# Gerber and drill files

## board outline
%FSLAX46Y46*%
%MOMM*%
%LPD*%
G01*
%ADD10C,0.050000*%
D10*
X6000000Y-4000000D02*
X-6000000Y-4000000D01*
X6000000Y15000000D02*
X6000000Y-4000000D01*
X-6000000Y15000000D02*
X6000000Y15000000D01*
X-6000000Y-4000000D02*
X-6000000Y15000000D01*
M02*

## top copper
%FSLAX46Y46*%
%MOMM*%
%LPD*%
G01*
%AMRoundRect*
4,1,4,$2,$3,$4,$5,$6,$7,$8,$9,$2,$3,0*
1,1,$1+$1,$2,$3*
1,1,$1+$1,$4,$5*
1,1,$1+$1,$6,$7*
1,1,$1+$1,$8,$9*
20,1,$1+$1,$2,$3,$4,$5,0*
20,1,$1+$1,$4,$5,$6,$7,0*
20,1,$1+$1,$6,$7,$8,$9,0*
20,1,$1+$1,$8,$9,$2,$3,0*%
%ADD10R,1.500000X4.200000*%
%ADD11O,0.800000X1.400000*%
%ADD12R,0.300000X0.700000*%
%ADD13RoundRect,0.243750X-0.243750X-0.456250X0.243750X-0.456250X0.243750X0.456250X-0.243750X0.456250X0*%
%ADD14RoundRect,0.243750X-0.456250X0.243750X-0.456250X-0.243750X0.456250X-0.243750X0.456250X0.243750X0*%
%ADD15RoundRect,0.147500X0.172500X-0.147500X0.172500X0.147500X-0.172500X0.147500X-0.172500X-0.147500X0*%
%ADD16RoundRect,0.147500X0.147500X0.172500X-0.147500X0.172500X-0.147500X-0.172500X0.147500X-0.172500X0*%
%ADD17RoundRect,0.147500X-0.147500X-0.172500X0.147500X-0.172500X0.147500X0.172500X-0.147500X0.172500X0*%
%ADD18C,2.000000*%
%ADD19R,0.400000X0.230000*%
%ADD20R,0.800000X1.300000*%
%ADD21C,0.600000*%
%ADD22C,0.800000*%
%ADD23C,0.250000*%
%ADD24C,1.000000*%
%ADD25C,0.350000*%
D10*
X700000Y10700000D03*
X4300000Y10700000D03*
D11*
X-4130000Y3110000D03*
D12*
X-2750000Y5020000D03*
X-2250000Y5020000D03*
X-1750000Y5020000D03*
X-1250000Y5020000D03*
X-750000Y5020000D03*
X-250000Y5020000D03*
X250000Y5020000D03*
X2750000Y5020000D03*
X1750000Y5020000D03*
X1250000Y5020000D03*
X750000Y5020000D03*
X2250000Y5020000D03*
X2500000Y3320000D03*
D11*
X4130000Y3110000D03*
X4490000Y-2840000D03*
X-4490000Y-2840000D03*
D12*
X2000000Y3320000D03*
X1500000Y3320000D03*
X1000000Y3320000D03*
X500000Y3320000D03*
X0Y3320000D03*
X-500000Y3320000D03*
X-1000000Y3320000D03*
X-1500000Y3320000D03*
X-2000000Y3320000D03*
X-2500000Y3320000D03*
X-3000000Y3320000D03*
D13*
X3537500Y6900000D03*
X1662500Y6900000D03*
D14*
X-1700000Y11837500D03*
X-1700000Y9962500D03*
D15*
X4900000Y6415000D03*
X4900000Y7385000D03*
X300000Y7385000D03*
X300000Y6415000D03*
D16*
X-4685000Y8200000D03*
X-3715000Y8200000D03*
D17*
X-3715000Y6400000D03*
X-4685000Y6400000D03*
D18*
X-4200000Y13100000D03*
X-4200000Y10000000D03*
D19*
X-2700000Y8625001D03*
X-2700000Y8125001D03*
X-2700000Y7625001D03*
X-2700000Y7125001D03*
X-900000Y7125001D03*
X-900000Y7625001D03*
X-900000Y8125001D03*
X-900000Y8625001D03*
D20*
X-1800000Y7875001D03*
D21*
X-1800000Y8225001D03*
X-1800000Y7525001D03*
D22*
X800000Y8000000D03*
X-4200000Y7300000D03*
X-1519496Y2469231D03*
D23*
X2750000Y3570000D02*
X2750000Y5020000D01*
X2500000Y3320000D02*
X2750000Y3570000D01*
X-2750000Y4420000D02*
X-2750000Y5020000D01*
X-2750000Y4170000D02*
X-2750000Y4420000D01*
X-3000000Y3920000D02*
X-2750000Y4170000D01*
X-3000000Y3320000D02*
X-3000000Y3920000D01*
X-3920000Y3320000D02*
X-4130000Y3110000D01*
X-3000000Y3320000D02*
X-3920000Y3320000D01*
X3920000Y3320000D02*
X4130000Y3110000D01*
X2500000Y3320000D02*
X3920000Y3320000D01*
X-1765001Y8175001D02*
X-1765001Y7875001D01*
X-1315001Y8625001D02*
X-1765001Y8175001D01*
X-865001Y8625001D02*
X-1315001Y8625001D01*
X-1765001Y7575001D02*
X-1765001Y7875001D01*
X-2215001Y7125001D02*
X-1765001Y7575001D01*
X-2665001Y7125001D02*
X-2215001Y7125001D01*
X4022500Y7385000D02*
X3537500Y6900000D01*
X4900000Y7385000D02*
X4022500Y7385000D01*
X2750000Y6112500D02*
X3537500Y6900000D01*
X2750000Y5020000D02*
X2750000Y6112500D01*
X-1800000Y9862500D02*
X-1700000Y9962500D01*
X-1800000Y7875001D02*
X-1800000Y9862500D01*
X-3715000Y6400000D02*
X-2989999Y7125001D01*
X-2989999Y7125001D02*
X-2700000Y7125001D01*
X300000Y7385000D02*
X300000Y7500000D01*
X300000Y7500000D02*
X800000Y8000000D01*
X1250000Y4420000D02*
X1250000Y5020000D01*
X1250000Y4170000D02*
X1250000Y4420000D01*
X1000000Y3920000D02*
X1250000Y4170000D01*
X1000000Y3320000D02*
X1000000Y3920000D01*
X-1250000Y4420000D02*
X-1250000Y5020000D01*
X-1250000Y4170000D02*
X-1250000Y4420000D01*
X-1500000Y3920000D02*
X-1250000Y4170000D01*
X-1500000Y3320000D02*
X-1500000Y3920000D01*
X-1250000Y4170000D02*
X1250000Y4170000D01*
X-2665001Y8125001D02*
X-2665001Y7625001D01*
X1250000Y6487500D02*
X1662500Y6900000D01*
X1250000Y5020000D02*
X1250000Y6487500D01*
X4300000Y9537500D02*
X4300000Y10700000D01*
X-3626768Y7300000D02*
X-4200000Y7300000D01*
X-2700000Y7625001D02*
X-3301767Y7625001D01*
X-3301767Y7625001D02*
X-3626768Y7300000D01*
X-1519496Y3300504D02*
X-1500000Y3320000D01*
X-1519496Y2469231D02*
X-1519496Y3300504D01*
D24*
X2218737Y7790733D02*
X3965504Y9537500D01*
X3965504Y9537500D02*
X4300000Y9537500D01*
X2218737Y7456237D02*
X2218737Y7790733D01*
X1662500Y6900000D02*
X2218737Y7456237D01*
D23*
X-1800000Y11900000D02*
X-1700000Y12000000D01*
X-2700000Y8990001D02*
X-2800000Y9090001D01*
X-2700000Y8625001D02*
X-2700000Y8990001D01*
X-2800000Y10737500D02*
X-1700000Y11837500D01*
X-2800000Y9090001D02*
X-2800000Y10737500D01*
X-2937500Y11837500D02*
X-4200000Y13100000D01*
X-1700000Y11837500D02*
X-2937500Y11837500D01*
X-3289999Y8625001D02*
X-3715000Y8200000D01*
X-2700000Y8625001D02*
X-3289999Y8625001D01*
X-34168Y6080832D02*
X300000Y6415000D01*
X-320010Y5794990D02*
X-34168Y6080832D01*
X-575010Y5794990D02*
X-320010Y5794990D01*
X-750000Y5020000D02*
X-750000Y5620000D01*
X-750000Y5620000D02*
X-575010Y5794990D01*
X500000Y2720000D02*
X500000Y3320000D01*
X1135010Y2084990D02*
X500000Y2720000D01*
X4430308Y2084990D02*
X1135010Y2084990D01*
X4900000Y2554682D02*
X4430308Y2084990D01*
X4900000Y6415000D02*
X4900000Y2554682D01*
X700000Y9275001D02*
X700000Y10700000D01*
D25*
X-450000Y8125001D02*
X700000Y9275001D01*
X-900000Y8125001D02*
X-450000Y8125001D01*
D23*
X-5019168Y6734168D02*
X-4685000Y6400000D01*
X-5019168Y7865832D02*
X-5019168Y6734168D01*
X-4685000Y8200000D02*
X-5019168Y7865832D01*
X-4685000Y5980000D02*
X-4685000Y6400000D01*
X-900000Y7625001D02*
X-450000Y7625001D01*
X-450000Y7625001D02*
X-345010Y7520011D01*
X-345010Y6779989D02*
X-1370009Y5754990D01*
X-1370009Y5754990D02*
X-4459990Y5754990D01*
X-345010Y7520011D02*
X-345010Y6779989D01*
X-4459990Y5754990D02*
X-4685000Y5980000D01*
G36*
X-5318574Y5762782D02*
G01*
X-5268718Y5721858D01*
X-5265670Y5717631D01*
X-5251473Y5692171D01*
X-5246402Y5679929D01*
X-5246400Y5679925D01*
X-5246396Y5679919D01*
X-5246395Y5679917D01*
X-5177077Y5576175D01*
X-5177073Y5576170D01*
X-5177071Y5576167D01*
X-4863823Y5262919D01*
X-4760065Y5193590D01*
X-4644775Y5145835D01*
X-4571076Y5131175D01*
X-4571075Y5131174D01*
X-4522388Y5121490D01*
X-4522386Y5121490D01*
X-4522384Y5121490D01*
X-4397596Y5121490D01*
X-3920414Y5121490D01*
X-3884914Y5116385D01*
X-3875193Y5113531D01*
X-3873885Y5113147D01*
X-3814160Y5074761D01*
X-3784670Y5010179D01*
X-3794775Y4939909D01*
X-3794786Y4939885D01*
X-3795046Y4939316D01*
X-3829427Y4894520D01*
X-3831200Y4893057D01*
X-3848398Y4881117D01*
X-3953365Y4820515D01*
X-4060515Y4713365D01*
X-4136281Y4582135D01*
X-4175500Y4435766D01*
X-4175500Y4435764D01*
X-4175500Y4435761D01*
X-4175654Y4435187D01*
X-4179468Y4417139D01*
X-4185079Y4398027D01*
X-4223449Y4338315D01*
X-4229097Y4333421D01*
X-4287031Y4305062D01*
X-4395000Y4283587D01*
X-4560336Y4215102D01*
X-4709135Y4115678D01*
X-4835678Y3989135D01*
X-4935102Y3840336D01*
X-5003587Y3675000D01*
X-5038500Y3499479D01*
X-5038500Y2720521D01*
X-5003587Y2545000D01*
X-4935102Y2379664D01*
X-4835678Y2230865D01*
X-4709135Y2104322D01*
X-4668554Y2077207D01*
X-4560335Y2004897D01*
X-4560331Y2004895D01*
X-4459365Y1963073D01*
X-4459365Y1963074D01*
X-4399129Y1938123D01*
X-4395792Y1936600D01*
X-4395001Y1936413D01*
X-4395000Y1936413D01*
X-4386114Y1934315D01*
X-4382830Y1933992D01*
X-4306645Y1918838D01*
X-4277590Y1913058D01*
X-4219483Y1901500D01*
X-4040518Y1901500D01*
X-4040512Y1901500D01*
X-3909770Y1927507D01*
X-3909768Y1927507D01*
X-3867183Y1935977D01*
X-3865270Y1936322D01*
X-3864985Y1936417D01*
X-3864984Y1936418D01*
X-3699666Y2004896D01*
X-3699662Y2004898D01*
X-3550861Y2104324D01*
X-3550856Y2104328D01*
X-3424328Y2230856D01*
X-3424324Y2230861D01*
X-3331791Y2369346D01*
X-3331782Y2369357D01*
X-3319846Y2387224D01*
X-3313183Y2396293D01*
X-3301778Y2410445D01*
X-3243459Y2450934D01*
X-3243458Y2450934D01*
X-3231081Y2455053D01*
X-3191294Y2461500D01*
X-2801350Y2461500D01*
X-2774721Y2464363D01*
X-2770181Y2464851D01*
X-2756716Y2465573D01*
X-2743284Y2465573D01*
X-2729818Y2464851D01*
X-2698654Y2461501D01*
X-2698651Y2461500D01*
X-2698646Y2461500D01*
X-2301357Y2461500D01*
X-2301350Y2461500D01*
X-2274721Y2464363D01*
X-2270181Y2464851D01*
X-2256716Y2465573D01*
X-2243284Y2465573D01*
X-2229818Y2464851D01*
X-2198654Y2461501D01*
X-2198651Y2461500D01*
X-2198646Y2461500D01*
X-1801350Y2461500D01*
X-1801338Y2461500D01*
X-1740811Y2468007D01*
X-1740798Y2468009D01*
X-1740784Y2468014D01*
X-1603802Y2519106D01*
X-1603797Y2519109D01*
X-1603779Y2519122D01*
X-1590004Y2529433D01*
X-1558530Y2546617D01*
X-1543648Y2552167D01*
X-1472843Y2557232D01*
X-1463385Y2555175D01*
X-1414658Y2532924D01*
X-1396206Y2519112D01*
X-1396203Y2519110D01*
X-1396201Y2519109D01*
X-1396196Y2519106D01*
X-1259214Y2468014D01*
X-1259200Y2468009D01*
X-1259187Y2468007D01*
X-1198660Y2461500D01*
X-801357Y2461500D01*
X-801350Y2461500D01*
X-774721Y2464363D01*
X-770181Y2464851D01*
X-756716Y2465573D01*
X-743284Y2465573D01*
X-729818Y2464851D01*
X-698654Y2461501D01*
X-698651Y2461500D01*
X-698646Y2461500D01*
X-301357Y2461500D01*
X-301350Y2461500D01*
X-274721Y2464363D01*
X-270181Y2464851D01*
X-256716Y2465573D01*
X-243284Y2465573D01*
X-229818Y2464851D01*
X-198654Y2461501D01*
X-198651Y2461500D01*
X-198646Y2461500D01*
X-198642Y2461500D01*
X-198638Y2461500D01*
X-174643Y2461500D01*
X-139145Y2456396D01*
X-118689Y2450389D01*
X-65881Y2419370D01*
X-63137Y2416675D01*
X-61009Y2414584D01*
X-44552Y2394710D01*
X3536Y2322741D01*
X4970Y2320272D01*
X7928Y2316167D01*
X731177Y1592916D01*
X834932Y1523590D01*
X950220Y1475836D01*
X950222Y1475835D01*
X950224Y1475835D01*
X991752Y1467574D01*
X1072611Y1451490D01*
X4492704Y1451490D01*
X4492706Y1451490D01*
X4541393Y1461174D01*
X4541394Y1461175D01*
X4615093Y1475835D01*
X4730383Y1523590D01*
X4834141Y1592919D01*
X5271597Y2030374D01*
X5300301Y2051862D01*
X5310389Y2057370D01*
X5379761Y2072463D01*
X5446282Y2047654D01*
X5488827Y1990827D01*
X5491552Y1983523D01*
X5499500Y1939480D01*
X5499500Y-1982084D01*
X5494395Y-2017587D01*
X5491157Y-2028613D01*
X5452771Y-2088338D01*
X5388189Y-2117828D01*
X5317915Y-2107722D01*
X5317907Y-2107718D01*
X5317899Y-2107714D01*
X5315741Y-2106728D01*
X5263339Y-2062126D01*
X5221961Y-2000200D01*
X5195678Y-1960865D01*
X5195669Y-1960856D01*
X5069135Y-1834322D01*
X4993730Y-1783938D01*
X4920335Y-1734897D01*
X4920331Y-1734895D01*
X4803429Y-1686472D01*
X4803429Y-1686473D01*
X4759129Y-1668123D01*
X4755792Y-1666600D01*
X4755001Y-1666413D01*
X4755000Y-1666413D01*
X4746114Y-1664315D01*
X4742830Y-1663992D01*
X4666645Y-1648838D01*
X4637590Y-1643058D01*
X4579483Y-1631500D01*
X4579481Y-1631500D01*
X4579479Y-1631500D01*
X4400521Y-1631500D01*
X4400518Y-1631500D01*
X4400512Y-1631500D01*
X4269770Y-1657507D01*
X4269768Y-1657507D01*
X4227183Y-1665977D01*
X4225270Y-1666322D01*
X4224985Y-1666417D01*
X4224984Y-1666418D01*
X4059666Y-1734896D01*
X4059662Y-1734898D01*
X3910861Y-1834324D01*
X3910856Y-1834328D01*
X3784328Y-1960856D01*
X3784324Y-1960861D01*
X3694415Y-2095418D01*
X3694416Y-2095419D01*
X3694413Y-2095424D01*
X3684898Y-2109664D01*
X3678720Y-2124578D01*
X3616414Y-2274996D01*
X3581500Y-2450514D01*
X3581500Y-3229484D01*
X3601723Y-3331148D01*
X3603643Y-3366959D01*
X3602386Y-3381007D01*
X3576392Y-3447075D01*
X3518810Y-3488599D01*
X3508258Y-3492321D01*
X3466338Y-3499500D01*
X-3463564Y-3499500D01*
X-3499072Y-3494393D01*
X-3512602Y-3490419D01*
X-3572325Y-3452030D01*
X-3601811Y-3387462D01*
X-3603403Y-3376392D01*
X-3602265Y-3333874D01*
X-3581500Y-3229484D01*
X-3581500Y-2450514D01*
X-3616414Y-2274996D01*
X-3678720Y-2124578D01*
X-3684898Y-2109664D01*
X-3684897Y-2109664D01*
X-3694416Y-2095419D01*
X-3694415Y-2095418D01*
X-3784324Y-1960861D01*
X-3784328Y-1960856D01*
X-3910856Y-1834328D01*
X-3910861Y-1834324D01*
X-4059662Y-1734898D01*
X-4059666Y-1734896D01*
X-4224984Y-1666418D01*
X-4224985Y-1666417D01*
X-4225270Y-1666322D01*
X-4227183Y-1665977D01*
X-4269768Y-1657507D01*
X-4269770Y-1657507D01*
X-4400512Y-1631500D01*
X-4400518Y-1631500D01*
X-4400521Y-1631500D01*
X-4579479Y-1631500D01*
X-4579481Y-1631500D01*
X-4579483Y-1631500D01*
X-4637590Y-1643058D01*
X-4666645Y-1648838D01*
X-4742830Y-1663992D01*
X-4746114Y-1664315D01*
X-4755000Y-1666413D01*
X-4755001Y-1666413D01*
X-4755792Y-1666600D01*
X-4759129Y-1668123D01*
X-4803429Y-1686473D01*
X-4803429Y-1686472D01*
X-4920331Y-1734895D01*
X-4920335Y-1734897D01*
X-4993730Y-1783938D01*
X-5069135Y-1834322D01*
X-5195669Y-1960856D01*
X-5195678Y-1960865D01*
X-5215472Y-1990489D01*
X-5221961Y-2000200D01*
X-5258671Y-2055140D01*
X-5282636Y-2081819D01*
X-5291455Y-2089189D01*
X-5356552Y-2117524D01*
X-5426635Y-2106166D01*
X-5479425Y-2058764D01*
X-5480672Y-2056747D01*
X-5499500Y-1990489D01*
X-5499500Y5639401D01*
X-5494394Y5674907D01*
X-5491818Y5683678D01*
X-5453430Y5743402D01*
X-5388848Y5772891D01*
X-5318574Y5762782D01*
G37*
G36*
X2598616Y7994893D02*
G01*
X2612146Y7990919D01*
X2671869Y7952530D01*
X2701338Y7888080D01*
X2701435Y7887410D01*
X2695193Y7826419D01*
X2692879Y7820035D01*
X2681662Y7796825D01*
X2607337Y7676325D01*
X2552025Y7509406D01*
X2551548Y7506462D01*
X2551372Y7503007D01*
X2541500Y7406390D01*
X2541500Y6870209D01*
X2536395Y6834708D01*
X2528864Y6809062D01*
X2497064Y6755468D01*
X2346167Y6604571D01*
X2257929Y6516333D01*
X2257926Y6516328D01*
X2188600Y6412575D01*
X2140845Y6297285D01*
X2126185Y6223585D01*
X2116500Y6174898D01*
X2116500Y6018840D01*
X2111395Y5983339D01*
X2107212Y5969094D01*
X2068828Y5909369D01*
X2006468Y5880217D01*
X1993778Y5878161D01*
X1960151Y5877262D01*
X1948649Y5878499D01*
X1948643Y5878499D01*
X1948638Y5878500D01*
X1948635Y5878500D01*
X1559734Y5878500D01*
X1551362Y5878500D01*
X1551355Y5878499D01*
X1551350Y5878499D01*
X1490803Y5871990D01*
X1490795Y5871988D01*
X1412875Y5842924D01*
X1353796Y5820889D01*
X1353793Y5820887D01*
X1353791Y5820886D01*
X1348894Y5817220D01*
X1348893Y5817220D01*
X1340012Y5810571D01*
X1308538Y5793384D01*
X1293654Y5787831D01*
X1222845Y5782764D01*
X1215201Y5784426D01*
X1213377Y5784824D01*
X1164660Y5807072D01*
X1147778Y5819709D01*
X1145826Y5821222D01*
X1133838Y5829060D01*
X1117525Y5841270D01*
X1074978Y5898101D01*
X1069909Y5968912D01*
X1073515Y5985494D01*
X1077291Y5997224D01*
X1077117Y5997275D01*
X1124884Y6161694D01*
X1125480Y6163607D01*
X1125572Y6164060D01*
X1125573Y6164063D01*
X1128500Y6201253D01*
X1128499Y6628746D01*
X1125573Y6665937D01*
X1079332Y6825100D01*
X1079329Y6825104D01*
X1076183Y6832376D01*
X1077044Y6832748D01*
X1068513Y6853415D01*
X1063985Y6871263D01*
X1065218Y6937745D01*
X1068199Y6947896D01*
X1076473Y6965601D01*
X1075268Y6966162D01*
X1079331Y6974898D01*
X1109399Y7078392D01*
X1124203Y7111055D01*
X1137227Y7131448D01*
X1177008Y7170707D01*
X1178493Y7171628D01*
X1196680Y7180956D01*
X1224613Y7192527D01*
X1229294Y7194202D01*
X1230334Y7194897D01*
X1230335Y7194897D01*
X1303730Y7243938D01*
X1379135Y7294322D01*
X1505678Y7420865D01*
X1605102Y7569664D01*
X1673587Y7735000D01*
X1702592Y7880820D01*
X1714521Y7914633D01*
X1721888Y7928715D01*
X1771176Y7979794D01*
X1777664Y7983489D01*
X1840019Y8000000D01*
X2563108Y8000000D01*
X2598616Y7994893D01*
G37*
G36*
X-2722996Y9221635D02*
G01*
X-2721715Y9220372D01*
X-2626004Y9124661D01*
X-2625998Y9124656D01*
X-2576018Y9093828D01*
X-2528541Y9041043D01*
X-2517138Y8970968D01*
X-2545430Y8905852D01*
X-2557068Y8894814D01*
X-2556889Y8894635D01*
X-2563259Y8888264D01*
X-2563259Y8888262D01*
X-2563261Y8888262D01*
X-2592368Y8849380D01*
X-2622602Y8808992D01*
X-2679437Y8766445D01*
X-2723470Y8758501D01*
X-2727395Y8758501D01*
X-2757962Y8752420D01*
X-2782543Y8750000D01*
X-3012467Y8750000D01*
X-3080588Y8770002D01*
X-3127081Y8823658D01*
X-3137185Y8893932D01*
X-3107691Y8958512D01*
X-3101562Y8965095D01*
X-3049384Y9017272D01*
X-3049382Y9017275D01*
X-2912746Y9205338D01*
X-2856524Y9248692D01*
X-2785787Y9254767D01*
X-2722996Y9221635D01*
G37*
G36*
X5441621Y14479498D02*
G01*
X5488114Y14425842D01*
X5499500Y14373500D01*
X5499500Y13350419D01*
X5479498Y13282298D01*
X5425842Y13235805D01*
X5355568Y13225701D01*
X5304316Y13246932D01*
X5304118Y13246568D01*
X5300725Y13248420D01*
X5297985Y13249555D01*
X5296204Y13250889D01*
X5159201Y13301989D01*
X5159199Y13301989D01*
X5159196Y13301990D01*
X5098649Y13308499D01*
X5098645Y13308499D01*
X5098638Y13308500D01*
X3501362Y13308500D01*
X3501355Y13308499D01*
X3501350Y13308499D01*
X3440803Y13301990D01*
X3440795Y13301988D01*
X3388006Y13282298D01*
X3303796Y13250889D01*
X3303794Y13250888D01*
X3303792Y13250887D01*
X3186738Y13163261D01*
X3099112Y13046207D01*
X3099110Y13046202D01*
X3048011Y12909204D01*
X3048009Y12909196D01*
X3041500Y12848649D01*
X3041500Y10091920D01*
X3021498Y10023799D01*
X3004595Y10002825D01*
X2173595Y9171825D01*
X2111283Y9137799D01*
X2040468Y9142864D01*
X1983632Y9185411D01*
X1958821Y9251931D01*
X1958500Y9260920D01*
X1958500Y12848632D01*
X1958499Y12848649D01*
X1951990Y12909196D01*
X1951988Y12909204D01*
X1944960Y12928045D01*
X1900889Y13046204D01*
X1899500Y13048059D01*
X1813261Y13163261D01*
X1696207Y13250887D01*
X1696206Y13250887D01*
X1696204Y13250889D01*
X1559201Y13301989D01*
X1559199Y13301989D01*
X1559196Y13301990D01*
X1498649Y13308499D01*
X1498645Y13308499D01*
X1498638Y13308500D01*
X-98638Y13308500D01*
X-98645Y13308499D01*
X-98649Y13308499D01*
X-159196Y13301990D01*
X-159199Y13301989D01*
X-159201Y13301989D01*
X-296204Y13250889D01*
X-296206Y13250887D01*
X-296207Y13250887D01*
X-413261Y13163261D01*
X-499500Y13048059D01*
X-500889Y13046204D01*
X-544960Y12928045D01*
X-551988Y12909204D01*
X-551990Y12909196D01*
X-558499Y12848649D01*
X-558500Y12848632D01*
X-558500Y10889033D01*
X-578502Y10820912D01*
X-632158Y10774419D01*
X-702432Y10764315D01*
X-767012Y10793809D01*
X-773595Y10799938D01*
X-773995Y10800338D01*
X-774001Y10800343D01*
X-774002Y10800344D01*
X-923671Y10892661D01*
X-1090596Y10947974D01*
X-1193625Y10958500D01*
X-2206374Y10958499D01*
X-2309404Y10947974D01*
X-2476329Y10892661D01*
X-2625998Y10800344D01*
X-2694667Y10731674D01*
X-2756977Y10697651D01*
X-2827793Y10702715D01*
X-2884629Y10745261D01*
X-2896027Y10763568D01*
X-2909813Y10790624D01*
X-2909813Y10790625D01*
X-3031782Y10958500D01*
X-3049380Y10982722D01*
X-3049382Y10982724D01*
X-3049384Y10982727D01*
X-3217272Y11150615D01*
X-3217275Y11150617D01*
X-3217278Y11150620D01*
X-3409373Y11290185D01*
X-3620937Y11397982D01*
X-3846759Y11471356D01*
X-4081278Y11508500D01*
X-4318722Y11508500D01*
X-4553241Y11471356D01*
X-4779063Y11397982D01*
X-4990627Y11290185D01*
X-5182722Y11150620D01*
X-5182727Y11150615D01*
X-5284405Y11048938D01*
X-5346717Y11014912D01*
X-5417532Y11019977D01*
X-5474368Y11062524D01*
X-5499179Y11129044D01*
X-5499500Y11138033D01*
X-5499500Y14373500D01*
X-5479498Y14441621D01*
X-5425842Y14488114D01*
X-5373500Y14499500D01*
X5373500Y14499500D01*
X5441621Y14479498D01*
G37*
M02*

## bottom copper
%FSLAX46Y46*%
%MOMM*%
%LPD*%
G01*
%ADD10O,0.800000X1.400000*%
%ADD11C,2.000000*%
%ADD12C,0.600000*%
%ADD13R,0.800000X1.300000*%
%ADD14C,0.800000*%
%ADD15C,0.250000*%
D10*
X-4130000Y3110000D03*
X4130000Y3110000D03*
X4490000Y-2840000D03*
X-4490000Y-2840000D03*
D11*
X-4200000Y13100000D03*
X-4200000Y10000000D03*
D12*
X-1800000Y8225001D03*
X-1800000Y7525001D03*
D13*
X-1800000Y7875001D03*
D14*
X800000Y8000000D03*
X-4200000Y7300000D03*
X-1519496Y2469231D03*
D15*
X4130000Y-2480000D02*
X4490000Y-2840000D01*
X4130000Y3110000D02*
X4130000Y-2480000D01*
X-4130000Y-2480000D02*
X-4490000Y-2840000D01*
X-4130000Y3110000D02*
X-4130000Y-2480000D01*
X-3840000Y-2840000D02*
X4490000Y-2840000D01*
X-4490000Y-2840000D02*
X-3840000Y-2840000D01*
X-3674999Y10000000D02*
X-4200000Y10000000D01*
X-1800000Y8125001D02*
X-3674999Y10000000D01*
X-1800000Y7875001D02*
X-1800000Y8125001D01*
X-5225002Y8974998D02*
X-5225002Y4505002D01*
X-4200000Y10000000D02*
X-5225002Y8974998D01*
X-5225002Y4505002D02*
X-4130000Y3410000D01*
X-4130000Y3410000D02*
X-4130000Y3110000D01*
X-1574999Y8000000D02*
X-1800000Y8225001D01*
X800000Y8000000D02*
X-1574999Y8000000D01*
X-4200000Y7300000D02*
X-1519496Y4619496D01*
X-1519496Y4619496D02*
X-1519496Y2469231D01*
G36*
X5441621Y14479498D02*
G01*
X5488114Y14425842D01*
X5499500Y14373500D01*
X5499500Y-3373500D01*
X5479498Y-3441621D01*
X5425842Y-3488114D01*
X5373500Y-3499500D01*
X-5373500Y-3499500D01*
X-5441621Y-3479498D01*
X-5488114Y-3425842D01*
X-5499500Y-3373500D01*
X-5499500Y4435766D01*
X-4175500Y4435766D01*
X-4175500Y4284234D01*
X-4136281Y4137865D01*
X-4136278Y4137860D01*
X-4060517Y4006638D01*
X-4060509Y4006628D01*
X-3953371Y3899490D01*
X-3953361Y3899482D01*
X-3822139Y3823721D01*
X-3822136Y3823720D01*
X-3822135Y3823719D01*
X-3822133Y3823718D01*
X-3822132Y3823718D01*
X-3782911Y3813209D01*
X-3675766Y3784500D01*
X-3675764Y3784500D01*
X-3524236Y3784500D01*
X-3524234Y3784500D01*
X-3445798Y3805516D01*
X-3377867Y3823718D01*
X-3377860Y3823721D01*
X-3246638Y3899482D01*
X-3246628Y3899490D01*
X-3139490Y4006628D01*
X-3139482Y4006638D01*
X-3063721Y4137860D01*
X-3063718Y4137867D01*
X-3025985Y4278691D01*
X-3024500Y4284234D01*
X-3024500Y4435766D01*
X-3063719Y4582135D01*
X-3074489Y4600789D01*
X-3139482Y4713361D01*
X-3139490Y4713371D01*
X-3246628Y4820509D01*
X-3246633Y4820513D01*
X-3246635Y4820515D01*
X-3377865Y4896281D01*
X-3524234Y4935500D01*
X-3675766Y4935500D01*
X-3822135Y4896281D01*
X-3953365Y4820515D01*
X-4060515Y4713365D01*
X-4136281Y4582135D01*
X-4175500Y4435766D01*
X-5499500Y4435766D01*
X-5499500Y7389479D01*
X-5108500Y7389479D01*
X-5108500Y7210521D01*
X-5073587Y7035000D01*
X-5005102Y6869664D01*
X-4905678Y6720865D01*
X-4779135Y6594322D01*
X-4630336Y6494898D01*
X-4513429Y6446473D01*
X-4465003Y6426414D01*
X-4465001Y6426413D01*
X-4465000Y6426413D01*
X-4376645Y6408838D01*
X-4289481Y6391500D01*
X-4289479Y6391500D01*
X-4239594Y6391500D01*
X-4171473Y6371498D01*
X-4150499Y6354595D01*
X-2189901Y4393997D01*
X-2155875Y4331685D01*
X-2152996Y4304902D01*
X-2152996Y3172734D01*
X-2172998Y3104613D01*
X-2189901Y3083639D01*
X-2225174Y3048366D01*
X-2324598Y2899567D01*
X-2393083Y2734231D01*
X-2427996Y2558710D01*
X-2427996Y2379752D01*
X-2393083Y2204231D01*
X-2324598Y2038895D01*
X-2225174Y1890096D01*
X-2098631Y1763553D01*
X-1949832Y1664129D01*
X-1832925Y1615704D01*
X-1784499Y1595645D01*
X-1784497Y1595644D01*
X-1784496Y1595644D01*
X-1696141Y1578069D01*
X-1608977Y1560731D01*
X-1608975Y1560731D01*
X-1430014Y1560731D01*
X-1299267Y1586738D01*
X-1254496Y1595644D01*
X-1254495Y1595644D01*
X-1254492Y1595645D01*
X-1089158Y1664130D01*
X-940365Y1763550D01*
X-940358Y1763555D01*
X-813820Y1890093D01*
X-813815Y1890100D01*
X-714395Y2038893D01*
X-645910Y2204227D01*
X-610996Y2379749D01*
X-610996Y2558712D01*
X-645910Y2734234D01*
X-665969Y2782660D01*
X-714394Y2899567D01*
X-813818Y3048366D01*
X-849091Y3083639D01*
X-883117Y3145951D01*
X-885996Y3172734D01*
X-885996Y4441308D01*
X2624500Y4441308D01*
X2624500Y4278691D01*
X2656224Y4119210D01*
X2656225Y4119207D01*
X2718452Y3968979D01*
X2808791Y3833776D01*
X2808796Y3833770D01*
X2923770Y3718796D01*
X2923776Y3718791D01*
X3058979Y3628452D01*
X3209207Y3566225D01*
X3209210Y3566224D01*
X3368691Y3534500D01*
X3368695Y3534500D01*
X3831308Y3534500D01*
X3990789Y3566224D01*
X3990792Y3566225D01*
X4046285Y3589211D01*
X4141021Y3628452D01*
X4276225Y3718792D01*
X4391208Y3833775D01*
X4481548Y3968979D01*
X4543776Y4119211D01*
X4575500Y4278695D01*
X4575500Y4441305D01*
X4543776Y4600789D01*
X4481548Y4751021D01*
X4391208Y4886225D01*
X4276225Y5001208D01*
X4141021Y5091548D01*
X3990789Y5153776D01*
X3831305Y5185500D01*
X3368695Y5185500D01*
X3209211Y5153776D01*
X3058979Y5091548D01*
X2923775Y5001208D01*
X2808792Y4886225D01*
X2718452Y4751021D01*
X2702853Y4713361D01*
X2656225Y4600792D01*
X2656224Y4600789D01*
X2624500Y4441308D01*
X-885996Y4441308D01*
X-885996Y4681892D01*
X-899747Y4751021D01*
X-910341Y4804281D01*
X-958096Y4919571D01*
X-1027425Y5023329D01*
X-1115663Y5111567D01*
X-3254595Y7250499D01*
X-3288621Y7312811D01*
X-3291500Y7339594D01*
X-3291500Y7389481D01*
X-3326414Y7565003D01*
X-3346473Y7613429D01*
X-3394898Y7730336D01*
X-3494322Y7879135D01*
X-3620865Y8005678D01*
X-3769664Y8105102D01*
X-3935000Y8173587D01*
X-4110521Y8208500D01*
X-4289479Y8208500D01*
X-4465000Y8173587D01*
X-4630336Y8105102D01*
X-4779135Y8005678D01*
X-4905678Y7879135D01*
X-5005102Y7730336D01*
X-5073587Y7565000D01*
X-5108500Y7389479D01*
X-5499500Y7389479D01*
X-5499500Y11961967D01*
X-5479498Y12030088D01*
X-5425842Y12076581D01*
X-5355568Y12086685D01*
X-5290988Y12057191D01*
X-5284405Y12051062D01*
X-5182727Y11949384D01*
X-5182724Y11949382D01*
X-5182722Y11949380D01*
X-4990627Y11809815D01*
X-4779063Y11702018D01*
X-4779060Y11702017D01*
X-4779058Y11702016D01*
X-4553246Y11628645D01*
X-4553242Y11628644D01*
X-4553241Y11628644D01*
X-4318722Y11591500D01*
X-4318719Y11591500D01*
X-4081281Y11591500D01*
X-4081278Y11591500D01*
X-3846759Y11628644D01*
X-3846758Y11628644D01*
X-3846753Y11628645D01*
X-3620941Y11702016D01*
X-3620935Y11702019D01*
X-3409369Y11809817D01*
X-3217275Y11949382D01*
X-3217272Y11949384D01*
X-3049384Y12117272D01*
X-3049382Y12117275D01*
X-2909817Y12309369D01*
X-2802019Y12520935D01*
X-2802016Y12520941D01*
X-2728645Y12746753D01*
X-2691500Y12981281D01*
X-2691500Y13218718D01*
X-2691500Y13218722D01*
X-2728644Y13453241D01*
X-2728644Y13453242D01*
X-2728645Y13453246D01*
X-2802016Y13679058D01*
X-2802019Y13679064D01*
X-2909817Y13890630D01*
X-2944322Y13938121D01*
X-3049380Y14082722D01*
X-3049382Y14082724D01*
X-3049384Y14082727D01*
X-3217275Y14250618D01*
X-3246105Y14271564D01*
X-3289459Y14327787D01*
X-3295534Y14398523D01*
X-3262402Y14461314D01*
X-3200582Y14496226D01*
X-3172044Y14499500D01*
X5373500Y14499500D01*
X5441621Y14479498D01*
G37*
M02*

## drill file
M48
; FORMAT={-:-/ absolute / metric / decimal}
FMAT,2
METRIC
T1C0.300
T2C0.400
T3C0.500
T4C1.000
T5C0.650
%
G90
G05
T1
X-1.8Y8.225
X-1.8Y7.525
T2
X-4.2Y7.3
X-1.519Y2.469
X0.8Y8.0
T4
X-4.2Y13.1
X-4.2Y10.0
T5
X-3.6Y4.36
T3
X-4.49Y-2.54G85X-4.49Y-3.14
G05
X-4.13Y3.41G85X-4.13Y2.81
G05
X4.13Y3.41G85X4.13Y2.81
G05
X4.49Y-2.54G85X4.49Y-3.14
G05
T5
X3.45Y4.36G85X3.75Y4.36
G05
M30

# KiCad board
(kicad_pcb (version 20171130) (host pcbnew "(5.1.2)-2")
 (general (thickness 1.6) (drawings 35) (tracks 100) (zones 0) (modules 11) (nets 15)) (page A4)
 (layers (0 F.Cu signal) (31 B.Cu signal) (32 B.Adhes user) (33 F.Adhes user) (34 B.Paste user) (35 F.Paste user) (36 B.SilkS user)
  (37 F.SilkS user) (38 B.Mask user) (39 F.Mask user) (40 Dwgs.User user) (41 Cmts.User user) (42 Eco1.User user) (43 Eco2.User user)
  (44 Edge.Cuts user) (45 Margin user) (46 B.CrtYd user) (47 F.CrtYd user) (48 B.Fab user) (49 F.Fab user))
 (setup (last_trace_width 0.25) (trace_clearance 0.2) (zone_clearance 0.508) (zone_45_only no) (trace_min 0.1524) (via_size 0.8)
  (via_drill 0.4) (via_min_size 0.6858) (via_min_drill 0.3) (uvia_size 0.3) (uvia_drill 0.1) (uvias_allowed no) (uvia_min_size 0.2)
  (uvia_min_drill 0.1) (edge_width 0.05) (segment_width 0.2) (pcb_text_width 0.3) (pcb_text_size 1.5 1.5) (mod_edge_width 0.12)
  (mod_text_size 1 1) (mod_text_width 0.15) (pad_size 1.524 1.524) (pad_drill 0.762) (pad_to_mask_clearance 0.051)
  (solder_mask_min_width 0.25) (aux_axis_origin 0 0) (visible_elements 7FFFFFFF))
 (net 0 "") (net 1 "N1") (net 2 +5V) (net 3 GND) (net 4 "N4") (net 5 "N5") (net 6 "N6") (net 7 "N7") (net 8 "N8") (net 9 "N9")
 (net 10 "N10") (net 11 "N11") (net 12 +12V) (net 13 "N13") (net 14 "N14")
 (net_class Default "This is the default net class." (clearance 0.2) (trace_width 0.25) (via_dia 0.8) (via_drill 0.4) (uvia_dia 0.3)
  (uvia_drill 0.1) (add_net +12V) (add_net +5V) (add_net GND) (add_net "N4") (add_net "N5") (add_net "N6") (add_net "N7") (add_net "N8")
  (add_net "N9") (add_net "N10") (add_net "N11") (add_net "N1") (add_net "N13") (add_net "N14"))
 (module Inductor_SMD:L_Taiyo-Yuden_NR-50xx (layer F.Cu) (at 2.5 -10.7)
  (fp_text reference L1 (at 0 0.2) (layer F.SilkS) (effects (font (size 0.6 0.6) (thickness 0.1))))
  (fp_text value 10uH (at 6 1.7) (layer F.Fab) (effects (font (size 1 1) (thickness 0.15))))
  (pad 1 smd rect (at -1.8 0) (size 1.5 4.2) (layers F.Cu F.Paste F.Mask) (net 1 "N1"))
  (pad 2 smd rect (at 1.8 0) (size 1.5 4.2) (layers F.Cu F.Paste F.Mask) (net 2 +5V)))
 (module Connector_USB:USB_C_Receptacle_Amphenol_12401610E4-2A (layer F.Cu) (at 0 0)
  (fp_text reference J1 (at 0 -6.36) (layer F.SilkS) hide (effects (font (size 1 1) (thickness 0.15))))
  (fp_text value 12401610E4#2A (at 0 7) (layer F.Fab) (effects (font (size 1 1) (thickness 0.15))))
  (pad S1 thru_hole oval (at -4.13 -3.11) (size 0.8 1.4) (drill oval 0.5 1.1) (layers *.Cu *.Mask) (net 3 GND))
  (pad A1 smd rect (at -2.75 -5.02) (size 0.3 0.7) (layers F.Cu F.Paste F.Mask) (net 3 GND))
  (pad A2 smd rect (at -2.25 -5.02) (size 0.3 0.7) (layers F.Cu F.Paste F.Mask))
  (pad A3 smd rect (at -1.75 -5.02) (size 0.3 0.7) (layers F.Cu F.Paste F.Mask))
  (pad A4 smd rect (at -1.25 -5.02) (size 0.3 0.7) (layers F.Cu F.Paste F.Mask) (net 2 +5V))
  (pad A5 smd rect (at -0.75 -5.02) (size 0.3 0.7) (layers F.Cu F.Paste F.Mask) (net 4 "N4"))
  (pad A6 smd rect (at -0.25 -5.02) (size 0.3 0.7) (layers F.Cu F.Paste F.Mask) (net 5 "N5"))
  (pad A7 smd rect (at 0.25 -5.02) (size 0.3 0.7) (layers F.Cu F.Paste F.Mask) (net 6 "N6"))
  (pad A12 smd rect (at 2.75 -5.02) (size 0.3 0.7) (layers F.Cu F.Paste F.Mask) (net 3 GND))
  (pad A10 smd rect (at 1.75 -5.02) (size 0.3 0.7) (layers F.Cu F.Paste F.Mask))
  (pad A9 smd rect (at 1.25 -5.02) (size 0.3 0.7) (layers F.Cu F.Paste F.Mask) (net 2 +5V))
  (pad A8 smd rect (at 0.75 -5.02) (size 0.3 0.7) (layers F.Cu F.Paste F.Mask) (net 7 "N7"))
  (pad A11 smd rect (at 2.25 -5.02) (size 0.3 0.7) (layers F.Cu F.Paste F.Mask))
  (pad B1 smd rect (at 2.5 -3.32) (size 0.3 0.7) (layers F.Cu F.Paste F.Mask) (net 3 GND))
  (pad S1 thru_hole oval (at 4.13 -3.11) (size 0.8 1.4) (drill oval 0.5 1.1) (layers *.Cu *.Mask) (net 3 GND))
  (pad S1 thru_hole oval (at 4.49 2.84) (size 0.8 1.4) (drill oval 0.5 1.1) (layers *.Cu *.Mask) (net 3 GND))
  (pad S1 thru_hole oval (at -4.49 2.84) (size 0.8 1.4) (drill oval 0.5 1.1) (layers *.Cu *.Mask) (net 3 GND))
  (pad "" np_thru_hole oval (at 3.6 -4.36) (size 0.95 0.65) (drill oval 0.95 0.65) (layers *.Cu *.Mask))
  (pad "" np_thru_hole circle (at -3.6 -4.36) (size 0.65 0.65) (drill 0.65) (layers *.Cu *.Mask))
  (pad B2 smd rect (at 2 -3.32) (size 0.3 0.7) (layers F.Cu F.Paste F.Mask))
  (pad B3 smd rect (at 1.5 -3.32) (size 0.3 0.7) (layers F.Cu F.Paste F.Mask))
  (pad B4 smd rect (at 1 -3.32) (size 0.3 0.7) (layers F.Cu F.Paste F.Mask) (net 2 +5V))
  (pad B5 smd rect (at 0.5 -3.32) (size 0.3 0.7) (layers F.Cu F.Paste F.Mask) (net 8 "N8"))
  (pad B6 smd rect (at 0 -3.32) (size 0.3 0.7) (layers F.Cu F.Paste F.Mask) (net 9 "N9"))
  (pad B7 smd rect (at -0.5 -3.32) (size 0.3 0.7) (layers F.Cu F.Paste F.Mask) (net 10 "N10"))
  (pad B8 smd rect (at -1 -3.32) (size 0.3 0.7) (layers F.Cu F.Paste F.Mask) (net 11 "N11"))
  (pad B9 smd rect (at -1.5 -3.32) (size 0.3 0.7) (layers F.Cu F.Paste F.Mask) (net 2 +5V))
  (pad B10 smd rect (at -2 -3.32) (size 0.3 0.7) (layers F.Cu F.Paste F.Mask))
  (pad B11 smd rect (at -2.5 -3.32) (size 0.3 0.7) (layers F.Cu F.Paste F.Mask))
  (pad B12 smd rect (at -3 -3.32) (size 0.3 0.7) (layers F.Cu F.Paste F.Mask) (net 3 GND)))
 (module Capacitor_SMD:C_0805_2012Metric (layer F.Cu) (at 2.6 -6.9)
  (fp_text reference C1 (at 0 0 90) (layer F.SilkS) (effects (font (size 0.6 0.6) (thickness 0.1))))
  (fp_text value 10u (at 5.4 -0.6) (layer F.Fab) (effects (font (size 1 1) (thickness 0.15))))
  (pad 2 smd roundrect (at 0.9375 0) (size 0.975 1.4) (layers F.Cu F.Paste F.Mask) (roundrect_rratio 0.25) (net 3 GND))
  (pad 1 smd roundrect (at -0.9375 0) (size 0.975 1.4) (layers F.Cu F.Paste F.Mask) (roundrect_rratio 0.25) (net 2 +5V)))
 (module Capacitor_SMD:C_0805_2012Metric (layer F.Cu) (at -1.7 -10.9 270)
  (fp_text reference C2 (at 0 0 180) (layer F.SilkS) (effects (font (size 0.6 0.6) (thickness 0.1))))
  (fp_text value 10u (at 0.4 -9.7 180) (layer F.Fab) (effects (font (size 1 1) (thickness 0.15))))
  (pad 1 smd roundrect (at -0.9375 0 270) (size 0.975 1.4) (layers F.Cu F.Paste F.Mask) (roundrect_rratio 0.25) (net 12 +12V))
  (pad 2 smd roundrect (at 0.9375 0 270) (size 0.975 1.4) (layers F.Cu F.Paste F.Mask) (roundrect_rratio 0.25) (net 3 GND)))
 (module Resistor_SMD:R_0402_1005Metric (layer F.Cu) (at 4.9 -6.9 90)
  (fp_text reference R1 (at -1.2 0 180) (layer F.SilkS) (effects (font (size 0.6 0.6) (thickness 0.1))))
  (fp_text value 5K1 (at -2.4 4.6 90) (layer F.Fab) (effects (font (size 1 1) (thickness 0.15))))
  (pad 1 smd roundrect (at -0.485 0 90) (size 0.59 0.64) (layers F.Cu F.Paste F.Mask) (roundrect_rratio 0.25) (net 8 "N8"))
  (pad 2 smd roundrect (at 0.485 0 90) (size 0.59 0.64) (layers F.Cu F.Paste F.Mask) (roundrect_rratio 0.25) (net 3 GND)))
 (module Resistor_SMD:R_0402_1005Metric (layer F.Cu) (at 0.3 -6.9 90)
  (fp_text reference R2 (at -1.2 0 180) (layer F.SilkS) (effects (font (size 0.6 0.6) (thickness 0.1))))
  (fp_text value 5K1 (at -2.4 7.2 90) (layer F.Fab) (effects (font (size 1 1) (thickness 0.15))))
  (pad 2 smd roundrect (at 0.485 0 90) (size 0.59 0.64) (layers F.Cu F.Paste F.Mask) (roundrect_rratio 0.25) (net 3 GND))
  (pad 1 smd roundrect (at -0.485 0 90) (size 0.59 0.64) (layers F.Cu F.Paste F.Mask) (roundrect_rratio 0.25) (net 4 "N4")))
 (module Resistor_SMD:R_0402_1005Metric (layer F.Cu) (at -4.2 -8.2 180)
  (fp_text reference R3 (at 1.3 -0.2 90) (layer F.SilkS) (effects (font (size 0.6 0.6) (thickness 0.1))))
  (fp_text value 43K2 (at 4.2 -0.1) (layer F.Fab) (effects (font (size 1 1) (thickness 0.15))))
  (pad 2 smd roundrect (at 0.485 0 180) (size 0.59 0.64) (layers F.Cu F.Paste F.Mask) (roundrect_rratio 0.25) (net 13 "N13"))
  (pad 1 smd roundrect (at -0.485 0 180) (size 0.59 0.64) (layers F.Cu F.Paste F.Mask) (roundrect_rratio 0.25) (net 12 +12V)))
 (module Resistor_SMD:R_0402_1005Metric (layer F.Cu) (at -4.2 -6.4)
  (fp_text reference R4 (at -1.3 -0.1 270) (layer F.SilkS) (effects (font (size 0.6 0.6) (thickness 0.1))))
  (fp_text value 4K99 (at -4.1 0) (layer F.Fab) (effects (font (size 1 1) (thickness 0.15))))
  (pad 2 smd roundrect (at 0.485 0) (size 0.59 0.64) (layers F.Cu F.Paste F.Mask) (roundrect_rratio 0.25) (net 3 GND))
  (pad 1 smd roundrect (at -0.485 0) (size 0.59 0.64) (layers F.Cu F.Paste F.Mask) (roundrect_rratio 0.25) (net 13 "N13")))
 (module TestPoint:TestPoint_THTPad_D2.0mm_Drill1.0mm (layer F.Cu) (at -4.2 -13.1)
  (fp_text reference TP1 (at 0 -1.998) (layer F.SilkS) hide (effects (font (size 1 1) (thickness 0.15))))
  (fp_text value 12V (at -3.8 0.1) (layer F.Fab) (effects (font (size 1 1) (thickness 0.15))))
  (pad 1 thru_hole circle (at 0 0) (size 2 2) (drill 1) (layers *.Cu *.Mask) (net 12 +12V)))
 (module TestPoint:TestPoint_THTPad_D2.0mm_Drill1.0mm (layer F.Cu) (at -4.2 -10)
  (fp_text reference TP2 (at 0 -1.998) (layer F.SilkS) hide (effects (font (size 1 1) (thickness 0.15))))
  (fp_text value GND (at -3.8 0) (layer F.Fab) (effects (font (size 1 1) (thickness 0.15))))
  (pad 1 thru_hole circle (at 0 0) (size 2 2) (drill 1) (layers *.Cu *.Mask) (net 3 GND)))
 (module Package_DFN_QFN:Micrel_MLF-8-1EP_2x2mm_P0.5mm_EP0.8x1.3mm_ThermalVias (layer F.Cu) (at -1.8 -7.875001)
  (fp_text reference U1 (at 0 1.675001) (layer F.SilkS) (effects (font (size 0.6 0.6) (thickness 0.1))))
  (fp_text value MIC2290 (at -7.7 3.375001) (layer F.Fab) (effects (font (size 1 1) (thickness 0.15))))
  (pad 1 smd rect (at -0.9 -0.75) (size 0.4 0.23) (layers F.Cu F.Paste F.Mask) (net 12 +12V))
  (pad 2 smd rect (at -0.9 -0.25) (size 0.4 0.23) (layers F.Cu F.Paste F.Mask) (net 2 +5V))
  (pad 3 smd rect (at -0.9 0.25) (size 0.4 0.23) (layers F.Cu F.Paste F.Mask) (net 2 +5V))
  (pad 4 smd rect (at -0.9 0.75) (size 0.4 0.23) (layers F.Cu F.Paste F.Mask) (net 3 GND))
  (pad 5 smd rect (at 0.9 0.75) (size 0.4 0.23) (layers F.Cu F.Paste F.Mask) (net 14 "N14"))
  (pad 6 smd rect (at 0.9 0.25) (size 0.4 0.23) (layers F.Cu F.Paste F.Mask) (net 13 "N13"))
  (pad 7 smd rect (at 0.9 -0.25) (size 0.4 0.23) (layers F.Cu F.Paste F.Mask) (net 1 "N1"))
  (pad 8 smd rect (at 0.9 -0.75) (size 0.4 0.23) (layers F.Cu F.Paste F.Mask) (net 3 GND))
  (pad 9 smd rect (at 0 0) (size 0.8 1.3) (layers F.Cu F.Mask) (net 3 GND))
  (pad 9 thru_hole circle (at 0 -0.35) (size 0.6 0.6) (drill 0.3) (layers *.Cu) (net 3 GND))
  (pad 9 thru_hole circle (at 0 0.35) (size 0.6 0.6) (drill 0.3) (layers *.Cu) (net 3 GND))
  (pad "" smd rect (at 0 -0.35) (size 0.55 0.55) (layers F.Paste))
  (pad "" smd rect (at 0 0.35) (size 0.55 0.55) (layers F.Paste))
  (pad 9 smd rect (at 0 0) (size 0.8 1.3) (layers B.Cu) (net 3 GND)))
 (gr_line (start 6 4) (end -6 4) (layer Edge.Cuts) (width 0.05))
 (gr_line (start 6 -15) (end 6 4) (layer Edge.Cuts) (width 0.05))
 (gr_line (start -6 -15) (end 6 -15) (layer Edge.Cuts) (width 0.05))
 (gr_line (start -6 4) (end -6 -15) (layer Edge.Cuts) (width 0.05))
 (segment (start 2.75 -3.57) (end 2.75 -5.02) (width 0.25) (layer F.Cu) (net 3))
 (segment (start 2.5 -3.32) (end 2.75 -3.57) (width 0.25) (layer F.Cu) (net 3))
 (segment (start -2.75 -4.42) (end -2.75 -5.02) (width 0.25) (layer F.Cu) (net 3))
 (segment (start -2.75 -4.17) (end -2.75 -4.42) (width 0.25) (layer F.Cu) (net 3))
 (segment (start -3 -3.92) (end -2.75 -4.17) (width 0.25) (layer F.Cu) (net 3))
 (segment (start -3 -3.32) (end -3 -3.92) (width 0.25) (layer F.Cu) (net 3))
 (segment (start -3.92 -3.32) (end -4.13 -3.11) (width 0.25) (layer F.Cu) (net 3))
 (segment (start -3 -3.32) (end -3.92 -3.32) (width 0.25) (layer F.Cu) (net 3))
 (segment (start 3.92 -3.32) (end 4.13 -3.11) (width 0.25) (layer F.Cu) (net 3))
 (segment (start 2.5 -3.32) (end 3.92 -3.32) (width 0.25) (layer F.Cu) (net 3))
 (segment (start 4.13 2.48) (end 4.49 2.84) (width 0.25) (layer B.Cu) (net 3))
 (segment (start 4.13 -3.11) (end 4.13 2.48) (width 0.25) (layer B.Cu) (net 3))
 (segment (start -4.13 2.48) (end -4.49 2.84) (width 0.25) (layer B.Cu) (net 3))
 (segment (start -4.13 -3.11) (end -4.13 2.48) (width 0.25) (layer B.Cu) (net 3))
 (segment (start -3.84 2.84) (end 4.49 2.84) (width 0.25) (layer B.Cu) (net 3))
 (segment (start -4.49 2.84) (end -3.84 2.84) (width 0.25) (layer B.Cu) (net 3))
 (segment (start -1.765001 -8.175001) (end -1.765001 -7.875001) (width 0.25) (layer F.Cu) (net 3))
 (segment (start -1.315001 -8.625001) (end -1.765001 -8.175001) (width 0.25) (layer F.Cu) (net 3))
 (segment (start -0.865001 -8.625001) (end -1.315001 -8.625001) (width 0.25) (layer F.Cu) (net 3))
 (segment (start -1.765001 -7.575001) (end -1.765001 -7.875001) (width 0.25) (layer F.Cu) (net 3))
 (segment (start -2.215001 -7.125001) (end -1.765001 -7.575001) (width 0.25) (layer F.Cu) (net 3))
 (segment (start -2.665001 -7.125001) (end -2.215001 -7.125001) (width 0.25) (layer F.Cu) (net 3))
 (segment (start 4.0225 -7.385) (end 3.5375 -6.9) (width 0.25) (layer F.Cu) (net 3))
 (segment (start 4.9 -7.385) (end 4.0225 -7.385) (width 0.25) (layer F.Cu) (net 3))
 (segment (start 2.75 -6.1125) (end 3.5375 -6.9) (width 0.25) (layer F.Cu) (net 3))
 (segment (start 2.75 -5.02) (end 2.75 -6.1125) (width 0.25) (layer F.Cu) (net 3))
 (segment (start -3.674999 -10) (end -4.2 -10) (width 0.25) (layer B.Cu) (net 3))
 (segment (start -1.8 -8.125001) (end -3.674999 -10) (width 0.25) (layer B.Cu) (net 3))
 (segment (start -1.8 -7.875001) (end -1.8 -8.125001) (width 0.25) (layer B.Cu) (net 3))
 (segment (start -1.8 -9.8625) (end -1.7 -9.9625) (width 0.25) (layer F.Cu) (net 3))
 (segment (start -1.8 -7.875001) (end -1.8 -9.8625) (width 0.25) (layer F.Cu) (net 3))
 (segment (start -5.225002 -8.974998) (end -5.225002 -4.505002) (width 0.25) (layer B.Cu) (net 3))
 (segment (start -4.2 -10) (end -5.225002 -8.974998) (width 0.25) (layer B.Cu) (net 3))
 (segment (start -5.225002 -4.505002) (end -4.13 -3.41) (width 0.25) (layer B.Cu) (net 3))
 (segment (start -4.13 -3.41) (end -4.13 -3.11) (width 0.25) (layer B.Cu) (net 3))
 (segment (start -3.715 -6.4) (end -2.989999 -7.125001) (width 0.25) (layer F.Cu) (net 3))
 (segment (start -2.989999 -7.125001) (end -2.7 -7.125001) (width 0.25) (layer F.Cu) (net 3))
 (via (at 0.8 -8) (size 0.8) (drill 0.4) (layers F.Cu B.Cu) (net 3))
 (segment (start 0.3 -7.385) (end 0.3 -7.5) (width 0.25) (layer F.Cu) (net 3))
 (segment (start 0.3 -7.5) (end 0.8 -8) (width 0.25) (layer F.Cu) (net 3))
 (segment (start -1.574999 -8) (end -1.8 -8.225001) (width 0.25) (layer B.Cu) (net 3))
 (segment (start 0.8 -8) (end -1.574999 -8) (width 0.25) (layer B.Cu) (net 3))
 (segment (start 1.25 -4.42) (end 1.25 -5.02) (width 0.25) (layer F.Cu) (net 2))
 (segment (start 1.25 -4.17) (end 1.25 -4.42) (width 0.25) (layer F.Cu) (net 2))
 (segment (start 1 -3.92) (end 1.25 -4.17) (width 0.25) (layer F.Cu) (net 2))
 (segment (start 1 -3.32) (end 1 -3.92) (width 0.25) (layer F.Cu) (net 2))
 (segment (start -1.25 -4.42) (end -1.25 -5.02) (width 0.25) (layer F.Cu) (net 2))
 (segment (start -1.25 -4.17) (end -1.25 -4.42) (width 0.25) (layer F.Cu) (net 2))
 (segment (start -1.5 -3.92) (end -1.25 -4.17) (width 0.25) (layer F.Cu) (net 2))
 (segment (start -1.5 -3.32) (end -1.5 -3.92) (width 0.25) (layer F.Cu) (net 2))
 (segment (start -1.25 -4.17) (end 1.25 -4.17) (width 0.25) (layer F.Cu) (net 2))
 (segment (start -2.665001 -8.125001) (end -2.665001 -7.625001) (width 0.25) (layer F.Cu) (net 2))
 (segment (start 1.25 -6.4875) (end 1.6625 -6.9) (width 0.25) (layer F.Cu) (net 2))
 (segment (start 1.25 -5.02) (end 1.25 -6.4875) (width 0.25) (layer F.Cu) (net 2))
 (segment (start 4.3 -9.5375) (end 4.3 -10.7) (width 0.25) (layer F.Cu) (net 2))
 (via (at -4.2 -7.3) (size 0.8) (drill 0.4) (layers F.Cu B.Cu) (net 2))
 (segment (start -3.626768 -7.3) (end -4.2 -7.3) (width 0.25) (layer F.Cu) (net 2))
 (segment (start -2.7 -7.625001) (end -3.301767 -7.625001) (width 0.25) (layer F.Cu) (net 2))
 (segment (start -3.301767 -7.625001) (end -3.626768 -7.3) (width 0.25) (layer F.Cu) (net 2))
 (via (at -1.519496 -2.469231) (size 0.8) (drill 0.4) (layers F.Cu B.Cu) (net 2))
 (segment (start -4.2 -7.3) (end -1.519496 -4.619496) (width 0.25) (layer B.Cu) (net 2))
 (segment (start -1.519496 -4.619496) (end -1.519496 -2.469231) (width 0.25) (layer B.Cu) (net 2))
 (segment (start -1.519496 -3.300504) (end -1.5 -3.32) (width 0.25) (layer F.Cu) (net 2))
 (segment (start -1.519496 -2.469231) (end -1.519496 -3.300504) (width 0.25) (layer F.Cu) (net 2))
 (segment (start 2.218737 -7.790733) (end 3.965504 -9.5375) (width 1) (layer F.Cu) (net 2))
 (segment (start 3.965504 -9.5375) (end 4.3 -9.5375) (width 1) (layer F.Cu) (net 2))
 (segment (start 2.218737 -7.456237) (end 2.218737 -7.790733) (width 1) (layer F.Cu) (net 2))
 (segment (start 1.6625 -6.9) (end 2.218737 -7.456237) (width 1) (layer F.Cu) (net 2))
 (segment (start -1.8 -11.9) (end -1.7 -12) (width 0.25) (layer F.Cu) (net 12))
 (segment (start -2.7 -8.990001) (end -2.8 -9.090001) (width 0.25) (layer F.Cu) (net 12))
 (segment (start -2.7 -8.625001) (end -2.7 -8.990001) (width 0.25) (layer F.Cu) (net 12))
 (segment (start -2.8 -10.7375) (end -1.7 -11.8375) (width 0.25) (layer F.Cu) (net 12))
 (segment (start -2.8 -9.090001) (end -2.8 -10.7375) (width 0.25) (layer F.Cu) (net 12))
 (segment (start -2.9375 -11.8375) (end -4.2 -13.1) (width 0.25) (layer F.Cu) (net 12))
 (segment (start -1.7 -11.8375) (end -2.9375 -11.8375) (width 0.25) (layer F.Cu) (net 12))
 (segment (start -3.289999 -8.625001) (end -3.715 -8.2) (width 0.25) (layer F.Cu) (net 12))
 (segment (start -2.7 -8.625001) (end -3.289999 -8.625001) (width 0.25) (layer F.Cu) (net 12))
 (segment (start -0.034168 -6.080832) (end 0.3 -6.415) (width 0.25) (layer F.Cu) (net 4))
 (segment (start -0.32001 -5.79499) (end -0.034168 -6.080832) (width 0.25) (layer F.Cu) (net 4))
 (segment (start -0.57501 -5.79499) (end -0.32001 -5.79499) (width 0.25) (layer F.Cu) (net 4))
 (segment (start -0.75 -5.02) (end -0.75 -5.62) (width 0.25) (layer F.Cu) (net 4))
 (segment (start -0.75 -5.62) (end -0.57501 -5.79499) (width 0.25) (layer F.Cu) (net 4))
 (segment (start 0.5 -2.72) (end 0.5 -3.32) (width 0.25) (layer F.Cu) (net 8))
 (segment (start 1.13501 -2.08499) (end 0.5 -2.72) (width 0.25) (layer F.Cu) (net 8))
 (segment (start 4.430308 -2.08499) (end 1.13501 -2.08499) (width 0.25) (layer F.Cu) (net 8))
 (segment (start 4.9 -2.554682) (end 4.430308 -2.08499) (width 0.25) (layer F.Cu) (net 8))
 (segment (start 4.9 -6.415) (end 4.9 -2.554682) (width 0.25) (layer F.Cu) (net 8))
 (segment (start 0.7 -9.275001) (end 0.7 -10.7) (width 0.25) (layer F.Cu) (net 1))
 (segment (start -0.45 -8.125001) (end 0.7 -9.275001) (width 0.35) (layer F.Cu) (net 1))
 (segment (start -0.9 -8.125001) (end -0.45 -8.125001) (width 0.35) (layer F.Cu) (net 1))
 (segment (start -5.019168 -6.734168) (end -4.685 -6.4) (width 0.25) (layer F.Cu) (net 13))
 (segment (start -5.019168 -7.865832) (end -5.019168 -6.734168) (width 0.25) (layer F.Cu) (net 13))
 (segment (start -4.685 -8.2) (end -5.019168 -7.865832) (width 0.25) (layer F.Cu) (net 13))
 (segment (start -4.685 -5.98) (end -4.685 -6.4) (width 0.25) (layer F.Cu) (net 13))
 (segment (start -0.9 -7.625001) (end -0.45 -7.625001) (width 0.25) (layer F.Cu) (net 13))
 (segment (start -0.45 -7.625001) (end -0.34501 -7.520011) (width 0.25) (layer F.Cu) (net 13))
 (segment (start -0.34501 -6.779989) (end -1.370009 -5.75499) (width 0.25) (layer F.Cu) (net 13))
 (segment (start -1.370009 -5.75499) (end -4.45999 -5.75499) (width 0.25) (layer F.Cu) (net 13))
 (segment (start -0.34501 -7.520011) (end -0.34501 -6.779989) (width 0.25) (layer F.Cu) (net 13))
 (segment (start -4.45999 -5.75499) (end -4.685 -5.98) (width 0.25) (layer F.Cu) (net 13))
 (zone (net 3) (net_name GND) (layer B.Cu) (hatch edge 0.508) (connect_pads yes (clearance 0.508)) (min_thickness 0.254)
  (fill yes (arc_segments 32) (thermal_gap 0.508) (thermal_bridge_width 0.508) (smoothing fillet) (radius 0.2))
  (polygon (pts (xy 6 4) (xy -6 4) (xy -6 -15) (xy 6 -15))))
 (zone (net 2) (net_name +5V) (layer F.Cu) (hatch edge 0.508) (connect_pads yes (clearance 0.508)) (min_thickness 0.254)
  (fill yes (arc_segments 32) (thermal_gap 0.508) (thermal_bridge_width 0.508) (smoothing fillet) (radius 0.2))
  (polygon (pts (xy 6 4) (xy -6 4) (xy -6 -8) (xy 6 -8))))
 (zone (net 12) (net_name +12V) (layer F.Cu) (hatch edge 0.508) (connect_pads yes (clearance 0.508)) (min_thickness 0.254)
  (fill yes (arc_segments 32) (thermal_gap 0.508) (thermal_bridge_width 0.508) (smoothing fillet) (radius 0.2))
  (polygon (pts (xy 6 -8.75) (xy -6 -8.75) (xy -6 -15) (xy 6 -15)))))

